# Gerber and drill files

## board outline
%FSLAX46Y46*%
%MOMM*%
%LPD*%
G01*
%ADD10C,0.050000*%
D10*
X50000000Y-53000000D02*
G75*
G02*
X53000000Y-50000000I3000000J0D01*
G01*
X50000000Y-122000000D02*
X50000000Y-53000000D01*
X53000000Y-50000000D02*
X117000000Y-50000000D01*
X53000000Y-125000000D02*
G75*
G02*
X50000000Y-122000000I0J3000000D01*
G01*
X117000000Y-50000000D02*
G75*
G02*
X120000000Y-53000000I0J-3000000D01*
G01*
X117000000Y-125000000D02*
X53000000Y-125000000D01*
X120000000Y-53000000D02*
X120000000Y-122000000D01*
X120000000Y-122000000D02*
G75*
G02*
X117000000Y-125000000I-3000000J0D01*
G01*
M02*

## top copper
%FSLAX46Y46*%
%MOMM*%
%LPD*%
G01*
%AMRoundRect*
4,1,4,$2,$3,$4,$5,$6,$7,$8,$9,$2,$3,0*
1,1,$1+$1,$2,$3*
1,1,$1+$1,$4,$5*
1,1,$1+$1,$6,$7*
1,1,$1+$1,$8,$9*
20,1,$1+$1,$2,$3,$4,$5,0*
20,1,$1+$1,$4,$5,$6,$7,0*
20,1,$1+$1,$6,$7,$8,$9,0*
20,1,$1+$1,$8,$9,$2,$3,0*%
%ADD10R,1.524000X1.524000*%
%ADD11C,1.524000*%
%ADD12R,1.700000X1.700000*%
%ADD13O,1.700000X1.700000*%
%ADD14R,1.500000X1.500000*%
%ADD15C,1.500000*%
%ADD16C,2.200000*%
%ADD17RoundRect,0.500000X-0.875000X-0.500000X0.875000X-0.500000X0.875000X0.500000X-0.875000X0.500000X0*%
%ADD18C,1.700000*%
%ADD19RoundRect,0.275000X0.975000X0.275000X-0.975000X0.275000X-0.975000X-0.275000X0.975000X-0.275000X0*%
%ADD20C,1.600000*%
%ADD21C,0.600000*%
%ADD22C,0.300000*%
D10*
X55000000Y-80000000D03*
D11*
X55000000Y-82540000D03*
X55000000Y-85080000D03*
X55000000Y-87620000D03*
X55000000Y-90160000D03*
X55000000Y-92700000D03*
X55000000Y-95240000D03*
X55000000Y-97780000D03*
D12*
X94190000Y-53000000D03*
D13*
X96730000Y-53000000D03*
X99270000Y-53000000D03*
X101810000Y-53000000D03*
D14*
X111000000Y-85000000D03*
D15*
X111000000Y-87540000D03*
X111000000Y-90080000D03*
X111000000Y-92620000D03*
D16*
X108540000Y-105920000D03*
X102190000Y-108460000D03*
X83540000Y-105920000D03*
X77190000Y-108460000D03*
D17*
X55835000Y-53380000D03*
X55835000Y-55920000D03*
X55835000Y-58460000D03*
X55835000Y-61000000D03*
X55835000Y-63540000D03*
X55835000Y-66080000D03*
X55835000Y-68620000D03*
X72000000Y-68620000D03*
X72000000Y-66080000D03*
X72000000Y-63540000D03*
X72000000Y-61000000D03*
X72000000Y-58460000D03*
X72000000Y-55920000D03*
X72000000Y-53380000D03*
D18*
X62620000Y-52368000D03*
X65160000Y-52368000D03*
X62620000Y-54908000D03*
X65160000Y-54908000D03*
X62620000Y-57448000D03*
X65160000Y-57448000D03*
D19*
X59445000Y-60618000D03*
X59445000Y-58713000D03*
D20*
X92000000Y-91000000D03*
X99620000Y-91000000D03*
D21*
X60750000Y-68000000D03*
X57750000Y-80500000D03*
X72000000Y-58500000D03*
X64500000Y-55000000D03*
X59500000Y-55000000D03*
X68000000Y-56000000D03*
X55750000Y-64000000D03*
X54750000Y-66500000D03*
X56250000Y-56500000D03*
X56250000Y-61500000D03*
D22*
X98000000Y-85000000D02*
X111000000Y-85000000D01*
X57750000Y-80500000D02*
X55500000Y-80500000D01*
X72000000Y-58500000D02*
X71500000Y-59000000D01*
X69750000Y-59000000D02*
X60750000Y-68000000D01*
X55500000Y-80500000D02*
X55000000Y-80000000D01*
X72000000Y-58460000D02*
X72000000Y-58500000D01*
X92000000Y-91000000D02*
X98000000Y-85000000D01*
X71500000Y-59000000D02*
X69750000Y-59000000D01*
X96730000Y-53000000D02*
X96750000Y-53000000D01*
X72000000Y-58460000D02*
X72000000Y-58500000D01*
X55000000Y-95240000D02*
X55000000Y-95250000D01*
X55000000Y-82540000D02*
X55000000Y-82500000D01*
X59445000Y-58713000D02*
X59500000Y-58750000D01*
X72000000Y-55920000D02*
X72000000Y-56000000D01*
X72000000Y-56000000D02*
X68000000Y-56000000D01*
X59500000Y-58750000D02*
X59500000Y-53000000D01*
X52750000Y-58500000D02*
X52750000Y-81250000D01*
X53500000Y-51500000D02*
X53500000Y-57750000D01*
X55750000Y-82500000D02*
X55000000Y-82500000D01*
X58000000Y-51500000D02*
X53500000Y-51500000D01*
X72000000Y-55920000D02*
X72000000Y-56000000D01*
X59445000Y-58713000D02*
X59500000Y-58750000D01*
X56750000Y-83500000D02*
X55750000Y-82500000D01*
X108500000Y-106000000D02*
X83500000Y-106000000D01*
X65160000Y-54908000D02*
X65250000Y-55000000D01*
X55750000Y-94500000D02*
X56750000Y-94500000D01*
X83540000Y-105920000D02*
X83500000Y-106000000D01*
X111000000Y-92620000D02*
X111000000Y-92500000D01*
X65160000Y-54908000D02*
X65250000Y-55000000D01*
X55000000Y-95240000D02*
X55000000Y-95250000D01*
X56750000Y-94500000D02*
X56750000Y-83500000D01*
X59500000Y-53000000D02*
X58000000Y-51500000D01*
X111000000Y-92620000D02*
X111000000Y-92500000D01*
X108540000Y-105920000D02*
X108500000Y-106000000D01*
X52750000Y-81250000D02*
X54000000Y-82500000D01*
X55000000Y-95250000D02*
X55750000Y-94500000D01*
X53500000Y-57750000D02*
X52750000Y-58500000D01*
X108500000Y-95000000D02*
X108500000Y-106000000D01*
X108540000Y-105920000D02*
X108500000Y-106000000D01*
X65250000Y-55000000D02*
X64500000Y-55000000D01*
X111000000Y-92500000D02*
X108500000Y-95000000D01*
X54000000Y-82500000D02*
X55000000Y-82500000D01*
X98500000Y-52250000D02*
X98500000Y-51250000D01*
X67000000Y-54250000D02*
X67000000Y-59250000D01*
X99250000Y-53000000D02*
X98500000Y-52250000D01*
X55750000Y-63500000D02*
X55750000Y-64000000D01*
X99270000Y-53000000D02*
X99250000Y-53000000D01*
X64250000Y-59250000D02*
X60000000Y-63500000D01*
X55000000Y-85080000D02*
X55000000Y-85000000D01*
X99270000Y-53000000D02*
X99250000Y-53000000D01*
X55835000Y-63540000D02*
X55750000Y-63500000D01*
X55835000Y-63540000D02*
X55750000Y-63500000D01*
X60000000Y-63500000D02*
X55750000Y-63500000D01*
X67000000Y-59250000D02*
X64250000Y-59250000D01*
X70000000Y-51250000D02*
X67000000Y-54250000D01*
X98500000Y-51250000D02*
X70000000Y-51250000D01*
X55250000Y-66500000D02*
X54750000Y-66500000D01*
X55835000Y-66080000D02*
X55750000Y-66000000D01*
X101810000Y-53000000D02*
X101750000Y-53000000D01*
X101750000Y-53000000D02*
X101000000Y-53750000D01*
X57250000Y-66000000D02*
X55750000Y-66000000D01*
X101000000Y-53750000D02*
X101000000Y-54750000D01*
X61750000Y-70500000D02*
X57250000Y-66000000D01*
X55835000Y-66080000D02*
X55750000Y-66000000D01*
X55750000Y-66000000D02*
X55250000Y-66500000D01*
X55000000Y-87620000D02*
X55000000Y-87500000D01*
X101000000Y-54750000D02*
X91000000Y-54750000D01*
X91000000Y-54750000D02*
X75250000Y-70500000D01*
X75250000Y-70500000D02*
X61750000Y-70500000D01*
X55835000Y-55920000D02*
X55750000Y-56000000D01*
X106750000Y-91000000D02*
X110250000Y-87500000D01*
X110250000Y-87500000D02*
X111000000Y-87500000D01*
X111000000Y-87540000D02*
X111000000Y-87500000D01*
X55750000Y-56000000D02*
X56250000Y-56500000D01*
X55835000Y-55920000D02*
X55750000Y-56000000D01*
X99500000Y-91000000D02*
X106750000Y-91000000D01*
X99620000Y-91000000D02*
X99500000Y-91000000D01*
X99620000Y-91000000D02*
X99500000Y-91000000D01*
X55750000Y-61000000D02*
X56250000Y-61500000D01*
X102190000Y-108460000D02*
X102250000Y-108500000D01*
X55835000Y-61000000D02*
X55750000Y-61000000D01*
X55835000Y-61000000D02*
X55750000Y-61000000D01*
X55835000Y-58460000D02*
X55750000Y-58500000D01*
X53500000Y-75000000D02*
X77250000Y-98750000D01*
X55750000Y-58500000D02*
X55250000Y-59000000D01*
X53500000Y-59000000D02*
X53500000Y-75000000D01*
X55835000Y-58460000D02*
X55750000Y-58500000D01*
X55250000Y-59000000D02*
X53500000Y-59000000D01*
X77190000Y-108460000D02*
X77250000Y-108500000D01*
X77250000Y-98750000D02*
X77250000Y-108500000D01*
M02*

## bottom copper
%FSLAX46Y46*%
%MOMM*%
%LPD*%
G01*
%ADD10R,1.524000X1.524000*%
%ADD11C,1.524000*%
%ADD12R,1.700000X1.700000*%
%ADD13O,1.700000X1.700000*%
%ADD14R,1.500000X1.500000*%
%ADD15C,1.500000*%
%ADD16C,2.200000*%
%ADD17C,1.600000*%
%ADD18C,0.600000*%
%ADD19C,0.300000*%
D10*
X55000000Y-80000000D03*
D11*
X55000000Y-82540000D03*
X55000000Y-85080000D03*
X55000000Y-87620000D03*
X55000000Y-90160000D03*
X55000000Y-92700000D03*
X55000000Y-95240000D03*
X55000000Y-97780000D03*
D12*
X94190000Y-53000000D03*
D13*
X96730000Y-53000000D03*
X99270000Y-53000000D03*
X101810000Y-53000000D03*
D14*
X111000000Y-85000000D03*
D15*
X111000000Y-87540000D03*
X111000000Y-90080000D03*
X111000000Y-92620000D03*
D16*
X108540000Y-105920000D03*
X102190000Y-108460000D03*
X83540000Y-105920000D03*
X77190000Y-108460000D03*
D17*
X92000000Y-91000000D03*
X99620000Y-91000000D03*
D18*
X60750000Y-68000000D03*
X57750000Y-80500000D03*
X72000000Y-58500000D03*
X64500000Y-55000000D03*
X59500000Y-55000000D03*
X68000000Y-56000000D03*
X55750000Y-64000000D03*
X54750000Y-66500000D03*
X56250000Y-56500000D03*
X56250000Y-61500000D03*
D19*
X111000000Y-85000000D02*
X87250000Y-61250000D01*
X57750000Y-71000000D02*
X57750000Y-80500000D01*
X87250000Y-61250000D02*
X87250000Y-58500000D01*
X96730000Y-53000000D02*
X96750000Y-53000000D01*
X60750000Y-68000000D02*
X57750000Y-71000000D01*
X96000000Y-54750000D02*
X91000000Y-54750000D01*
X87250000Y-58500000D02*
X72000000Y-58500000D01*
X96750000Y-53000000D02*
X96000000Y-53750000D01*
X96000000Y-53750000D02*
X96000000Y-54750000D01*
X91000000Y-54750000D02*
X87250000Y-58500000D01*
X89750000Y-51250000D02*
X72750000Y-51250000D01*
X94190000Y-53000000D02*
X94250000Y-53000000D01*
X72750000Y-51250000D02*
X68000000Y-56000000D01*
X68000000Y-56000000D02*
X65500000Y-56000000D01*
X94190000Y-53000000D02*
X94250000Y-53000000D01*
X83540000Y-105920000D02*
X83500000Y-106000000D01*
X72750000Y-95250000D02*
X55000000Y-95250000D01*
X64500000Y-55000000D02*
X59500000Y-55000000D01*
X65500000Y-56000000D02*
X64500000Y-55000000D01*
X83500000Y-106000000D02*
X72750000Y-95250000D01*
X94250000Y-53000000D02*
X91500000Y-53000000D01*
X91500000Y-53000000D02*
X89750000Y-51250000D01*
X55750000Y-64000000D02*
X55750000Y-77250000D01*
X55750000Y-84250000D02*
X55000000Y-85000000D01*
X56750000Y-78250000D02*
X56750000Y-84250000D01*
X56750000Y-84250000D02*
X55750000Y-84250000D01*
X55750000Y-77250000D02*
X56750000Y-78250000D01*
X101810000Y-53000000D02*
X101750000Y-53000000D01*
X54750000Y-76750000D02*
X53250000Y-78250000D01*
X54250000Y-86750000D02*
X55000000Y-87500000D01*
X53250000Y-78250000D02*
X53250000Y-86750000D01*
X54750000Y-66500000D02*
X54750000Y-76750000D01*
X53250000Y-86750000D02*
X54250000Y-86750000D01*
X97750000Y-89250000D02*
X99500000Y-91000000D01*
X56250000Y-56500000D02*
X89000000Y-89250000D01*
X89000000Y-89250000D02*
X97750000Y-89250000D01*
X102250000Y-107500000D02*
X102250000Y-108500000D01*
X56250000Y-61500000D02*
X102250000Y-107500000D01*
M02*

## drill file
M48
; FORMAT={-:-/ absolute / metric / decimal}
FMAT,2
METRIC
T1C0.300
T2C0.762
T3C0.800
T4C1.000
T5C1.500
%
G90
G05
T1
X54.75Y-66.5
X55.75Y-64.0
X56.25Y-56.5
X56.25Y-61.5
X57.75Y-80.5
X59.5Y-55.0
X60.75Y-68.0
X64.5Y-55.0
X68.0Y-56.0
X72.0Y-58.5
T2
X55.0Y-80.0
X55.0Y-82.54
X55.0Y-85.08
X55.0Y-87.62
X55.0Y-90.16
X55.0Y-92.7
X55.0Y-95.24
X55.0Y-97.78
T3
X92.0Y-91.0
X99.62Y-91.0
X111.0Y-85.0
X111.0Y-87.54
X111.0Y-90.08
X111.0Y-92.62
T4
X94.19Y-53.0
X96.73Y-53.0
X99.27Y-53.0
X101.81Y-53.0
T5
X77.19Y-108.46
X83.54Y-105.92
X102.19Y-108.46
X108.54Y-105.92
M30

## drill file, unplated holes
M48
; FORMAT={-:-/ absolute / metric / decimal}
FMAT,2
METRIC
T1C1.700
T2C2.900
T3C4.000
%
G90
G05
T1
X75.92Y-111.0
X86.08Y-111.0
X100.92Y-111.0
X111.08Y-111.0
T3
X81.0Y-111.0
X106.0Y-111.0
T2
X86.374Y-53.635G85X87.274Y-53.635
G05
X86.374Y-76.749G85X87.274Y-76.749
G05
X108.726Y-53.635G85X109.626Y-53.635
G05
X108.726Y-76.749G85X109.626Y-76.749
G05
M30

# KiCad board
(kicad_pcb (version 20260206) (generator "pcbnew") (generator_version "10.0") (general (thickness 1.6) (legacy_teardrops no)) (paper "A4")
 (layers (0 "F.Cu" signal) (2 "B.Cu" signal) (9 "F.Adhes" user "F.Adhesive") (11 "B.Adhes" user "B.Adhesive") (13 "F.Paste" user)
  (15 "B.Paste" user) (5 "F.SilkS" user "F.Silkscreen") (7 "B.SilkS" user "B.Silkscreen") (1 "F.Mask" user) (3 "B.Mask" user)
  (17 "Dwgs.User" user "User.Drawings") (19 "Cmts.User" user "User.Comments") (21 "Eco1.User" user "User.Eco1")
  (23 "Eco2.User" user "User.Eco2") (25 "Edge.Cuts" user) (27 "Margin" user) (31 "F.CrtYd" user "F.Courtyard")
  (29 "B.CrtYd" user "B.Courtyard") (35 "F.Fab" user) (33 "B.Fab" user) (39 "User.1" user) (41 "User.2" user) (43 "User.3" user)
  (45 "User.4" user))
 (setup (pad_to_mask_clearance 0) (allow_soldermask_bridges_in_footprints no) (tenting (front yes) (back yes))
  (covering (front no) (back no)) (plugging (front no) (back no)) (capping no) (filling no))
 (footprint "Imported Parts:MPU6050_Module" (layer "F.Cu") (at 55 80)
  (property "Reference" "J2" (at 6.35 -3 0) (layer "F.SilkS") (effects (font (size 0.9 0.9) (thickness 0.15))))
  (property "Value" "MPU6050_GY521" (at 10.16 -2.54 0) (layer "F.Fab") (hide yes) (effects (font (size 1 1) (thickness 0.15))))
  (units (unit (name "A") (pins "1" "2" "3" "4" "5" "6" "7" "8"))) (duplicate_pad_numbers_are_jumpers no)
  (pad "1" thru_hole rect (at 0 0) (size 1.524 1.524) (drill 0.762) (layers "*.Cu" "*.Mask") (remove_unused_layers no) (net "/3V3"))
  (pad "2" thru_hole circle (at 0 2.54) (size 1.524 1.524) (drill 0.762) (layers "*.Cu" "*.Mask") (remove_unused_layers no) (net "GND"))
  (pad "3" thru_hole circle (at 0 5.08) (size 1.524 1.524) (drill 0.762) (layers "*.Cu" "*.Mask") (remove_unused_layers no) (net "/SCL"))
  (pad "4" thru_hole circle (at 0 7.62) (size 1.524 1.524) (drill 0.762) (layers "*.Cu" "*.Mask") (remove_unused_layers no) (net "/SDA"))
  (pad "5" thru_hole circle (at 0 10.16) (size 1.524 1.524) (drill 0.762) (layers "*.Cu" "*.Mask") (remove_unused_layers no)
   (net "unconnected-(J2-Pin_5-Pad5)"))
  (pad "6" thru_hole circle (at 0 12.7) (size 1.524 1.524) (drill 0.762) (layers "*.Cu" "*.Mask") (remove_unused_layers no)
   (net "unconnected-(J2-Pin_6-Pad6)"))
  (pad "7" thru_hole circle (at 0 15.24) (size 1.524 1.524) (drill 0.762) (layers "*.Cu" "*.Mask") (remove_unused_layers no) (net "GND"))
  (pad "8" thru_hole circle (at 0 17.78) (size 1.524 1.524) (drill 0.762) (layers "*.Cu" "*.Mask") (remove_unused_layers no)
   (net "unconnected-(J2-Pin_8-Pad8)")))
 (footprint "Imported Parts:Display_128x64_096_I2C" (layer "F.Cu") (at 98 53)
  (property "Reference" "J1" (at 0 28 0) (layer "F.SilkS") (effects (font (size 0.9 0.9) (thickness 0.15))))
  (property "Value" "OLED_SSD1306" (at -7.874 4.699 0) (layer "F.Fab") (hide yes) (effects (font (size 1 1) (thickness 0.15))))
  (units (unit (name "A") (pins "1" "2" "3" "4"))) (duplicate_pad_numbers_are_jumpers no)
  (pad "" np_thru_hole oval (at -11.176 0.635) (size 3.8 2.9) (drill oval 3.8 2.9) (layers "*.Cu" "*.Mask"))
  (pad "" np_thru_hole oval (at -11.176 23.749) (size 3.8 2.9) (drill oval 3.8 2.9) (layers "*.Cu" "*.Mask"))
  (pad "" np_thru_hole oval (at 11.176 0.635) (size 3.8 2.9) (drill oval 3.8 2.9) (layers "*.Cu" "*.Mask"))
  (pad "" np_thru_hole oval (at 11.176 23.749) (size 3.8 2.9) (drill oval 3.8 2.9) (layers "*.Cu" "*.Mask"))
  (pad "1" thru_hole rect (at -3.81 0 90) (size 1.7 1.7) (drill 1) (layers "*.Cu" "*.Mask") (remove_unused_layers no) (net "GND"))
  (pad "2" thru_hole oval (at -1.27 0 90) (size 1.7 1.7) (drill 1) (layers "*.Cu" "*.Mask") (remove_unused_layers no) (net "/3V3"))
  (pad "3" thru_hole oval (at 1.27 0 90) (size 1.7 1.7) (drill 1) (layers "*.Cu" "*.Mask") (remove_unused_layers no) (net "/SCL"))
  (pad "4" thru_hole oval (at 3.81 0 90) (size 1.7 1.7) (drill 1) (layers "*.Cu" "*.Mask") (remove_unused_layers no) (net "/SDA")))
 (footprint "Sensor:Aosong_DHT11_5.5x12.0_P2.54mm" (layer "F.Cu") (at 111 85)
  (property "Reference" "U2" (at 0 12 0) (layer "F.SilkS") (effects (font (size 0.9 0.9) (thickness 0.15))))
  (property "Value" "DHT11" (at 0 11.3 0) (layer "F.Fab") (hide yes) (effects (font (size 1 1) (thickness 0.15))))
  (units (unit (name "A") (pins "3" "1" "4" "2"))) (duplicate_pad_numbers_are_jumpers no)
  (pad "1" thru_hole rect (at 0 0) (size 1.5 1.5) (drill 0.8) (layers "*.Cu" "*.Mask") (remove_unused_layers no) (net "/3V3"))
  (pad "2" thru_hole circle (at 0 2.54) (size 1.5 1.5) (drill 0.8) (layers "*.Cu" "*.Mask") (remove_unused_layers no) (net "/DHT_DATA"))
  (pad "3" thru_hole circle (at 0 5.08) (size 1.5 1.5) (drill 0.8) (layers "*.Cu" "*.Mask") (remove_unused_layers no)
   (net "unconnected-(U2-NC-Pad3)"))
  (pad "4" thru_hole circle (at 0 7.62) (size 1.5 1.5) (drill 0.8) (layers "*.Cu" "*.Mask") (remove_unused_layers no) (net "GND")))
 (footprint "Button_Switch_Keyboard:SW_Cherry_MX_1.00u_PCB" (layer "F.Cu") (at 108.54 105.92)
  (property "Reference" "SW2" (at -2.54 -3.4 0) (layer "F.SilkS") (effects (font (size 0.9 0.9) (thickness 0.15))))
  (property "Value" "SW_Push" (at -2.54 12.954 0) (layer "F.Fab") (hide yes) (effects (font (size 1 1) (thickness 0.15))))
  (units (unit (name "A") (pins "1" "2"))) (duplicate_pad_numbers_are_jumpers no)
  (pad "" np_thru_hole circle (at -7.62 5.08) (size 1.7 1.7) (drill 1.7) (layers "*.Cu" "*.Mask"))
  (pad "" np_thru_hole circle (at -2.54 5.08) (size 4 4) (drill 4) (layers "*.Cu" "*.Mask"))
  (pad "" np_thru_hole circle (at 2.54 5.08) (size 1.7 1.7) (drill 1.7) (layers "*.Cu" "*.Mask"))
  (pad "1" thru_hole circle (at 0 0) (size 2.2 2.2) (drill 1.5) (layers "*.Cu" "*.Mask") (remove_unused_layers no) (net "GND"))
  (pad "2" thru_hole circle (at -6.35 2.54) (size 2.2 2.2) (drill 1.5) (layers "*.Cu" "*.Mask") (remove_unused_layers no)
   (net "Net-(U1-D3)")))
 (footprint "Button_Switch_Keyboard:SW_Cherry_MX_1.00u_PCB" (layer "F.Cu") (at 83.54 105.92)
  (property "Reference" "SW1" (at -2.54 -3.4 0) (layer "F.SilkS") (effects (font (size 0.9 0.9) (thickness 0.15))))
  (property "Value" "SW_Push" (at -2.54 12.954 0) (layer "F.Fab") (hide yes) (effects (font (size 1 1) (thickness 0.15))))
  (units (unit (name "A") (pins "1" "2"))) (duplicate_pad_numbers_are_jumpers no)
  (pad "" np_thru_hole circle (at -7.62 5.08) (size 1.7 1.7) (drill 1.7) (layers "*.Cu" "*.Mask"))
  (pad "" np_thru_hole circle (at -2.54 5.08) (size 4 4) (drill 4) (layers "*.Cu" "*.Mask"))
  (pad "" np_thru_hole circle (at 2.54 5.08) (size 1.7 1.7) (drill 1.7) (layers "*.Cu" "*.Mask"))
  (pad "1" thru_hole circle (at 0 0) (size 2.2 2.2) (drill 1.5) (layers "*.Cu" "*.Mask") (remove_unused_layers no) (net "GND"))
  (pad "2" thru_hole circle (at -6.35 2.54) (size 2.2 2.2) (drill 1.5) (layers "*.Cu" "*.Mask") (remove_unused_layers no)
   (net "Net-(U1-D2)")))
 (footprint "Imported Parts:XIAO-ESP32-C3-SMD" (layer "F.Cu") (at 55 71.5)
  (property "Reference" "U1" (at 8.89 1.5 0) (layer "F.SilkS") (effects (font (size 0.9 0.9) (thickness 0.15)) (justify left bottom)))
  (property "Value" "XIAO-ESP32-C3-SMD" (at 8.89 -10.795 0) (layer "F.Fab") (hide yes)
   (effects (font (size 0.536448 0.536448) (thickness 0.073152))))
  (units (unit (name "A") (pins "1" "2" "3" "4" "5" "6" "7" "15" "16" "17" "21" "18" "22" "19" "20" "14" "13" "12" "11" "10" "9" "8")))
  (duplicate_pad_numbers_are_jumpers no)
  (pad "1" smd roundrect (at 0.835 -18.12) (size 2.75 2) (layers "F.Cu" "F.Mask" "F.Paste") (roundrect_rratio 0.25)
   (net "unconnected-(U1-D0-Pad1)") (solder_mask_margin 0.0508) (thermal_bridge_angle 45))
  (pad "2" smd roundrect (at 0.835 -15.58) (size 2.75 2) (layers "F.Cu" "F.Mask" "F.Paste") (roundrect_rratio 0.25) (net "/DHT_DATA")
   (solder_mask_margin 0.0508) (thermal_bridge_angle 45))
  (pad "3" smd roundrect (at 0.835 -13.04) (size 2.75 2) (layers "F.Cu" "F.Mask" "F.Paste") (roundrect_rratio 0.25) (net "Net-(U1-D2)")
   (solder_mask_margin 0.0508) (thermal_bridge_angle 45))
  (pad "4" smd roundrect (at 0.835 -10.5) (size 2.75 2) (layers "F.Cu" "F.Mask" "F.Paste") (roundrect_rratio 0.25) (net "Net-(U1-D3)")
   (solder_mask_margin 0.0508) (thermal_bridge_angle 45))
  (pad "5" smd roundrect (at 0.835 -7.96) (size 2.75 2) (layers "F.Cu" "F.Mask" "F.Paste") (roundrect_rratio 0.25) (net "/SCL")
   (solder_mask_margin 0.0508) (thermal_bridge_angle 45))
  (pad "6" smd roundrect (at 0.835 -5.42) (size 2.75 2) (layers "F.Cu" "F.Mask" "F.Paste") (roundrect_rratio 0.25) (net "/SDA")
   (solder_mask_margin 0.0508) (thermal_bridge_angle 45))
  (pad "7" smd roundrect (at 0.835 -2.88) (size 2.75 2) (layers "F.Cu" "F.Mask" "F.Paste") (roundrect_rratio 0.25)
   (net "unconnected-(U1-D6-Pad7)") (solder_mask_margin 0.0508) (thermal_bridge_angle 45))
  (pad "8" smd roundrect (at 17 -2.88) (size 2.75 2) (layers "F.Cu" "F.Mask" "F.Paste") (roundrect_rratio 0.25)
   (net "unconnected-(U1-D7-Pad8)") (solder_mask_margin 0.0508) (thermal_bridge_angle 45))
  (pad "9" smd roundrect (at 17 -5.42) (size 2.75 2) (layers "F.Cu" "F.Mask" "F.Paste") (roundrect_rratio 0.25)
   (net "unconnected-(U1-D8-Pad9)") (solder_mask_margin 0.0508) (thermal_bridge_angle 45))
  (pad "10" smd roundrect (at 17 -7.96) (size 2.75 2) (layers "F.Cu" "F.Mask" "F.Paste") (roundrect_rratio 0.25)
   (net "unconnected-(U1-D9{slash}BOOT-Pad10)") (solder_mask_margin 0.0508) (thermal_bridge_angle 45))
  (pad "11" smd roundrect (at 17 -10.5) (size 2.75 2) (layers "F.Cu" "F.Mask" "F.Paste") (roundrect_rratio 0.25)
   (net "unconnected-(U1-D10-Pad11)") (solder_mask_margin 0.0508) (thermal_bridge_angle 45))
  (pad "12" smd roundrect (at 17 -13.04) (size 2.75 2) (layers "F.Cu" "F.Mask" "F.Paste") (roundrect_rratio 0.25) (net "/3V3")
   (solder_mask_margin 0.0508) (thermal_bridge_angle 45))
  (pad "13" smd roundrect (at 17 -15.58) (size 2.75 2) (layers "F.Cu" "F.Mask" "F.Paste") (roundrect_rratio 0.25) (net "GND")
   (solder_mask_margin 0.0508) (thermal_bridge_angle 45))
  (pad "14" smd roundrect (at 17 -18.12) (size 2.75 2) (layers "F.Cu" "F.Mask" "F.Paste") (roundrect_rratio 0.25)
   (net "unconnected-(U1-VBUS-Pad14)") (solder_mask_margin 0.0508) (thermal_bridge_angle 45))
  (pad "15" smd circle (at 7.62 -19.132) (size 1.7 1.7) (layers "F.Cu" "F.Mask" "F.Paste") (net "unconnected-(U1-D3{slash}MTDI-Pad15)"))
  (pad "16" smd circle (at 10.16 -19.132) (size 1.7 1.7) (layers "F.Cu" "F.Mask" "F.Paste") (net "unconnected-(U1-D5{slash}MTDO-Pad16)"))
  (pad "17" smd circle (at 7.62 -16.592) (size 1.7 1.7) (layers "F.Cu" "F.Mask" "F.Paste") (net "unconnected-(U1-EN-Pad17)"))
  (pad "18" smd circle (at 10.16 -16.592) (size 1.7 1.7) (layers "F.Cu" "F.Mask" "F.Paste") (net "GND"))
  (pad "19" smd circle (at 7.62 -14.052) (size 1.7 1.7) (layers "F.Cu" "F.Mask" "F.Paste") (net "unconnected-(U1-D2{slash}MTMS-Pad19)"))
  (pad "20" smd circle (at 10.16 -14.052) (size 1.7 1.7) (layers "F.Cu" "F.Mask" "F.Paste") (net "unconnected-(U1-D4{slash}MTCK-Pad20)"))
  (pad "21" smd roundrect (at 4.445 -10.882 180) (size 2.5 1.1) (layers "F.Cu" "F.Mask" "F.Paste") (roundrect_rratio 0.25)
   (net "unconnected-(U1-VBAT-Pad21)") (thermal_bridge_angle 45))
  (pad "22" smd roundrect (at 4.445 -12.787 180) (size 2.5 1.1) (layers "F.Cu" "F.Mask" "F.Paste") (roundrect_rratio 0.25) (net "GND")
   (thermal_bridge_angle 45)))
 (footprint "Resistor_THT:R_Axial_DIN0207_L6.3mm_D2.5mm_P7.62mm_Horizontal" (layer "F.Cu") (at 92 91)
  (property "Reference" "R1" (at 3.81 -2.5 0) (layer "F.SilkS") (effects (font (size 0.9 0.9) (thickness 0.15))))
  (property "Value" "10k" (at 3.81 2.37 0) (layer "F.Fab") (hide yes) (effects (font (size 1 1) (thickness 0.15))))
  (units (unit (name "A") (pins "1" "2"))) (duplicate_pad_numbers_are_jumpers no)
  (pad "1" thru_hole circle (at 0 0) (size 1.6 1.6) (drill 0.8) (layers "*.Cu" "*.Mask") (remove_unused_layers no) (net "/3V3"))
  (pad "2" thru_hole circle (at 7.62 0) (size 1.6 1.6) (drill 0.8) (layers "*.Cu" "*.Mask") (remove_unused_layers no) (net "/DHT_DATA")))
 (gr_arc (start 50 53) (mid 50.87868 50.87868) (end 53 50) (stroke (width 0.05) (type default)) (layer "Edge.Cuts"))
 (gr_line (start 50 122) (end 50 53) (stroke (width 0.05) (type default)) (layer "Edge.Cuts"))
 (gr_line (start 53 50) (end 117 50) (stroke (width 0.05) (type default)) (layer "Edge.Cuts"))
 (gr_arc (start 53 125) (mid 50.87868 124.12132) (end 50 122) (stroke (width 0.05) (type default)) (layer "Edge.Cuts"))
 (gr_arc (start 117 50) (mid 119.12132 50.87868) (end 120 53) (stroke (width 0.05) (type default)) (layer "Edge.Cuts"))
 (gr_line (start 117 125) (end 53 125) (stroke (width 0.05) (type default)) (layer "Edge.Cuts"))
 (gr_line (start 120 53) (end 120 122) (stroke (width 0.05) (type default)) (layer "Edge.Cuts"))
 (gr_arc (start 120 122) (mid 119.12132 124.12132) (end 117 125) (stroke (width 0.05) (type default)) (layer "Edge.Cuts"))
 (segment (start 98 85) (end 111 85) (width 0.3) (layer "F.Cu") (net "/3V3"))
 (segment (start 57.75 80.5) (end 55.5 80.5) (width 0.3) (layer "F.Cu") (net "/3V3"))
 (segment (start 72 58.5) (end 71.5 59) (width 0.3) (layer "F.Cu") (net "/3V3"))
 (segment (start 69.75 59) (end 60.75 68) (width 0.3) (layer "F.Cu") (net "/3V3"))
 (segment (start 55.5 80.5) (end 55 80) (width 0.3) (layer "F.Cu") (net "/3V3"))
 (segment (start 72 58.46) (end 72 58.5) (width 0.3) (layer "F.Cu") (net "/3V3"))
 (segment (start 92 91) (end 98 85) (width 0.3) (layer "F.Cu") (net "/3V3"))
 (segment (start 71.5 59) (end 69.75 59) (width 0.3) (layer "F.Cu") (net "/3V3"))
 (segment (start 96.73 53) (end 96.75 53) (width 0.3) (layer "F.Cu") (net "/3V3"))
 (segment (start 72 58.46) (end 72 58.5) (width 0.3) (layer "F.Cu") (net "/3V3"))
 (via (at 60.75 68) (size 0.6) (drill 0.3) (layers "F.Cu" "B.Cu") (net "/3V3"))
 (via (at 57.75 80.5) (size 0.6) (drill 0.3) (layers "F.Cu" "B.Cu") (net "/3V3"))
 (via (at 72 58.5) (size 0.6) (drill 0.3) (layers "F.Cu" "B.Cu") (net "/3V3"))
 (segment (start 111 85) (end 87.25 61.25) (width 0.3) (layer "B.Cu") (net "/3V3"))
 (segment (start 57.75 71) (end 57.75 80.5) (width 0.3) (layer "B.Cu") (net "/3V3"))
 (segment (start 87.25 61.25) (end 87.25 58.5) (width 0.3) (layer "B.Cu") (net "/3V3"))
 (segment (start 96.73 53) (end 96.75 53) (width 0.3) (layer "B.Cu") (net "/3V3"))
 (segment (start 60.75 68) (end 57.75 71) (width 0.3) (layer "B.Cu") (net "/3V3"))
 (segment (start 96 54.75) (end 91 54.75) (width 0.3) (layer "B.Cu") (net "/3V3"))
 (segment (start 87.25 58.5) (end 72 58.5) (width 0.3) (layer "B.Cu") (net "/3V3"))
 (segment (start 96.75 53) (end 96 53.75) (width 0.3) (layer "B.Cu") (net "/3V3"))
 (segment (start 96 53.75) (end 96 54.75) (width 0.3) (layer "B.Cu") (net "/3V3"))
 (segment (start 91 54.75) (end 87.25 58.5) (width 0.3) (layer "B.Cu") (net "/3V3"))
 (segment (start 55 95.24) (end 55 95.25) (width 0.3) (layer "F.Cu") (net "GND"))
 (segment (start 55 82.54) (end 55 82.5) (width 0.3) (layer "F.Cu") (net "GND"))
 (segment (start 59.445 58.713) (end 59.5 58.75) (width 0.3) (layer "F.Cu") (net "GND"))
 (segment (start 72 55.92) (end 72 56) (width 0.3) (layer "F.Cu") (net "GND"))
 (segment (start 72 56) (end 68 56) (width 0.3) (layer "F.Cu") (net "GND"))
 (segment (start 59.5 58.75) (end 59.5 53) (width 0.3) (layer "F.Cu") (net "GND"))
 (segment (start 52.75 58.5) (end 52.75 81.25) (width 0.3) (layer "F.Cu") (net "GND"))
 (segment (start 53.5 51.5) (end 53.5 57.75) (width 0.3) (layer "F.Cu") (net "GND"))
 (segment (start 55.75 82.5) (end 55 82.5) (width 0.3) (layer "F.Cu") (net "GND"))
 (segment (start 58 51.5) (end 53.5 51.5) (width 0.3) (layer "F.Cu") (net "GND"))
 (segment (start 72 55.92) (end 72 56) (width 0.3) (layer "F.Cu") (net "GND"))
 (segment (start 59.445 58.713) (end 59.5 58.75) (width 0.3) (layer "F.Cu") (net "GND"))
 (segment (start 56.75 83.5) (end 55.75 82.5) (width 0.3) (layer "F.Cu") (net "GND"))
 (segment (start 108.5 106) (end 83.5 106) (width 0.3) (layer "F.Cu") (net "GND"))
 (segment (start 65.16 54.908) (end 65.25 55) (width 0.3) (layer "F.Cu") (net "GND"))
 (segment (start 55.75 94.5) (end 56.75 94.5) (width 0.3) (layer "F.Cu") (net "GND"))
 (segment (start 83.54 105.92) (end 83.5 106) (width 0.3) (layer "F.Cu") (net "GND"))
 (segment (start 111 92.62) (end 111 92.5) (width 0.3) (layer "F.Cu") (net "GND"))
 (segment (start 65.16 54.908) (end 65.25 55) (width 0.3) (layer "F.Cu") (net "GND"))
 (segment (start 55 95.24) (end 55 95.25) (width 0.3) (layer "F.Cu") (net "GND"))
 (segment (start 56.75 94.5) (end 56.75 83.5) (width 0.3) (layer "F.Cu") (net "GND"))
 (segment (start 59.5 53) (end 58 51.5) (width 0.3) (layer "F.Cu") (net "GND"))
 (segment (start 111 92.62) (end 111 92.5) (width 0.3) (layer "F.Cu") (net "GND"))
 (segment (start 108.54 105.92) (end 108.5 106) (width 0.3) (layer "F.Cu") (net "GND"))
 (segment (start 52.75 81.25) (end 54 82.5) (width 0.3) (layer "F.Cu") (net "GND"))
 (segment (start 55 95.25) (end 55.75 94.5) (width 0.3) (layer "F.Cu") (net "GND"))
 (segment (start 53.5 57.75) (end 52.75 58.5) (width 0.3) (layer "F.Cu") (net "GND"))
 (segment (start 108.5 95) (end 108.5 106) (width 0.3) (layer "F.Cu") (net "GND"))
 (segment (start 108.54 105.92) (end 108.5 106) (width 0.3) (layer "F.Cu") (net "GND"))
 (segment (start 65.25 55) (end 64.5 55) (width 0.3) (layer "F.Cu") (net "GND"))
 (segment (start 111 92.5) (end 108.5 95) (width 0.3) (layer "F.Cu") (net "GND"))
 (segment (start 54 82.5) (end 55 82.5) (width 0.3) (layer "F.Cu") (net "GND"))
 (via (at 64.5 55) (size 0.6) (drill 0.3) (layers "F.Cu" "B.Cu") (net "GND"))
 (via (at 59.5 55) (size 0.6) (drill 0.3) (layers "F.Cu" "B.Cu") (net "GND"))
 (via (at 68 56) (size 0.6) (drill 0.3) (layers "F.Cu" "B.Cu") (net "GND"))
 (segment (start 89.75 51.25) (end 72.75 51.25) (width 0.3) (layer "B.Cu") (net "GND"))
 (segment (start 94.19 53) (end 94.25 53) (width 0.3) (layer "B.Cu") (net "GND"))
 (segment (start 72.75 51.25) (end 68 56) (width 0.3) (layer "B.Cu") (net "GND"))
 (segment (start 68 56) (end 65.5 56) (width 0.3) (layer "B.Cu") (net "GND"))
 (segment (start 94.19 53) (end 94.25 53) (width 0.3) (layer "B.Cu") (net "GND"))
 (segment (start 83.54 105.92) (end 83.5 106) (width 0.3) (layer "B.Cu") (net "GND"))
 (segment (start 72.75 95.25) (end 55 95.25) (width 0.3) (layer "B.Cu") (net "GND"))
 (segment (start 64.5 55) (end 59.5 55) (width 0.3) (layer "B.Cu") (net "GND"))
 (segment (start 65.5 56) (end 64.5 55) (width 0.3) (layer "B.Cu") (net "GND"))
 (segment (start 83.5 106) (end 72.75 95.25) (width 0.3) (layer "B.Cu") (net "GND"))
 (segment (start 94.25 53) (end 91.5 53) (width 0.3) (layer "B.Cu") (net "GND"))
 (segment (start 91.5 53) (end 89.75 51.25) (width 0.3) (layer "B.Cu") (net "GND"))
 (segment (start 98.5 52.25) (end 98.5 51.25) (width 0.3) (layer "F.Cu") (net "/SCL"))
 (segment (start 67 54.25) (end 67 59.25) (width 0.3) (layer "F.Cu") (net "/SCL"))
 (segment (start 99.25 53) (end 98.5 52.25) (width 0.3) (layer "F.Cu") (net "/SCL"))
 (segment (start 55.75 63.5) (end 55.75 64) (width 0.3) (layer "F.Cu") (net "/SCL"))
 (segment (start 99.27 53) (end 99.25 53) (width 0.3) (layer "F.Cu") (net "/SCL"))
 (segment (start 64.25 59.25) (end 60 63.5) (width 0.3) (layer "F.Cu") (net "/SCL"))
 (segment (start 55 85.08) (end 55 85) (width 0.3) (layer "F.Cu") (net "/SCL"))
 (segment (start 99.27 53) (end 99.25 53) (width 0.3) (layer "F.Cu") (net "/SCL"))
 (segment (start 55.835 63.54) (end 55.75 63.5) (width 0.3) (layer "F.Cu") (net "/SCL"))
 (segment (start 55.835 63.54) (end 55.75 63.5) (width 0.3) (layer "F.Cu") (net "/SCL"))
 (segment (start 60 63.5) (end 55.75 63.5) (width 0.3) (layer "F.Cu") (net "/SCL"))
 (segment (start 67 59.25) (end 64.25 59.25) (width 0.3) (layer "F.Cu") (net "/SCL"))
 (segment (start 70 51.25) (end 67 54.25) (width 0.3) (layer "F.Cu") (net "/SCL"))
 (segment (start 98.5 51.25) (end 70 51.25) (width 0.3) (layer "F.Cu") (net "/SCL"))
 (via (at 55.75 64) (size 0.6) (drill 0.3) (layers "F.Cu" "B.Cu") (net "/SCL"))
 (segment (start 55.75 64) (end 55.75 77.25) (width 0.3) (layer "B.Cu") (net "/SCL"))
 (segment (start 55.75 84.25) (end 55 85) (width 0.3) (layer "B.Cu") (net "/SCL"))
 (segment (start 56.75 78.25) (end 56.75 84.25) (width 0.3) (layer "B.Cu") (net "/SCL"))
 (segment (start 56.75 84.25) (end 55.75 84.25) (width 0.3) (layer "B.Cu") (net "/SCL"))
 (segment (start 55.75 77.25) (end 56.75 78.25) (width 0.3) (layer "B.Cu") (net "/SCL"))
 (segment (start 55.25 66.5) (end 54.75 66.5) (width 0.3) (layer "F.Cu") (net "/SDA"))
 (segment (start 55.835 66.08) (end 55.75 66) (width 0.3) (layer "F.Cu") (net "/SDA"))
 (segment (start 101.81 53) (end 101.75 53) (width 0.3) (layer "F.Cu") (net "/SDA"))
 (segment (start 101.75 53) (end 101 53.75) (width 0.3) (layer "F.Cu") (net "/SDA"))
 (segment (start 57.25 66) (end 55.75 66) (width 0.3) (layer "F.Cu") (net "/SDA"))
 (segment (start 101 53.75) (end 101 54.75) (width 0.3) (layer "F.Cu") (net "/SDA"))
 (segment (start 61.75 70.5) (end 57.25 66) (width 0.3) (layer "F.Cu") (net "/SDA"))
 (segment (start 55.835 66.08) (end 55.75 66) (width 0.3) (layer "F.Cu") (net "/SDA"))
 (segment (start 55.75 66) (end 55.25 66.5) (width 0.3) (layer "F.Cu") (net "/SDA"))
 (segment (start 55 87.62) (end 55 87.5) (width 0.3) (layer "F.Cu") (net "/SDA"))
 (segment (start 101 54.75) (end 91 54.75) (width 0.3) (layer "F.Cu") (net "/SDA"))
 (segment (start 91 54.75) (end 75.25 70.5) (width 0.3) (layer "F.Cu") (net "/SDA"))
 (segment (start 75.25 70.5) (end 61.75 70.5) (width 0.3) (layer "F.Cu") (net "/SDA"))
 (via (at 54.75 66.5) (size 0.6) (drill 0.3) (layers "F.Cu" "B.Cu") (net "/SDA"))
 (segment (start 101.81 53) (end 101.75 53) (width 0.3) (layer "B.Cu") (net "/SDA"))
 (segment (start 54.75 76.75) (end 53.25 78.25) (width 0.3) (layer "B.Cu") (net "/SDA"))
 (segment (start 54.25 86.75) (end 55 87.5) (width 0.3) (layer "B.Cu") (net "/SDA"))
 (segment (start 53.25 78.25) (end 53.25 86.75) (width 0.3) (layer "B.Cu") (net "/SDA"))
 (segment (start 54.75 66.5) (end 54.75 76.75) (width 0.3) (layer "B.Cu") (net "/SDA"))
 (segment (start 53.25 86.75) (end 54.25 86.75) (width 0.3) (layer "B.Cu") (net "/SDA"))
 (segment (start 55.835 55.92) (end 55.75 56) (width 0.3) (layer "F.Cu") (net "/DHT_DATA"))
 (segment (start 106.75 91) (end 110.25 87.5) (width 0.3) (layer "F.Cu") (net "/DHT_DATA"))
 (segment (start 110.25 87.5) (end 111 87.5) (width 0.3) (layer "F.Cu") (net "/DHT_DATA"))
 (segment (start 111 87.54) (end 111 87.5) (width 0.3) (layer "F.Cu") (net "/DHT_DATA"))
 (segment (start 55.75 56) (end 56.25 56.5) (width 0.3) (layer "F.Cu") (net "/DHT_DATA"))
 (segment (start 55.835 55.92) (end 55.75 56) (width 0.3) (layer "F.Cu") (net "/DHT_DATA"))
 (segment (start 99.5 91) (end 106.75 91) (width 0.3) (layer "F.Cu") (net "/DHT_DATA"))
 (segment (start 99.62 91) (end 99.5 91) (width 0.3) (layer "F.Cu") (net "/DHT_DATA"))
 (segment (start 99.62 91) (end 99.5 91) (width 0.3) (layer "F.Cu") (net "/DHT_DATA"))
 (via (at 56.25 56.5) (size 0.6) (drill 0.3) (layers "F.Cu" "B.Cu") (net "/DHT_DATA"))
 (segment (start 97.75 89.25) (end 99.5 91) (width 0.3) (layer "B.Cu") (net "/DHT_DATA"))
 (segment (start 56.25 56.5) (end 89 89.25) (width 0.3) (layer "B.Cu") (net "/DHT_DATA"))
 (segment (start 89 89.25) (end 97.75 89.25) (width 0.3) (layer "B.Cu") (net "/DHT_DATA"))
 (segment (start 55.75 61) (end 56.25 61.5) (width 0.3) (layer "F.Cu") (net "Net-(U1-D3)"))
 (segment (start 102.19 108.46) (end 102.25 108.5) (width 0.3) (layer "F.Cu") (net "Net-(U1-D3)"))
 (segment (start 55.835 61) (end 55.75 61) (width 0.3) (layer "F.Cu") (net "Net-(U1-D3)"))
 (segment (start 55.835 61) (end 55.75 61) (width 0.3) (layer "F.Cu") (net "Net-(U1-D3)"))
 (via (at 56.25 61.5) (size 0.6) (drill 0.3) (layers "F.Cu" "B.Cu") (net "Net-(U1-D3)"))
 (segment (start 102.25 107.5) (end 102.25 108.5) (width 0.3) (layer "B.Cu") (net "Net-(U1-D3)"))
 (segment (start 56.25 61.5) (end 102.25 107.5) (width 0.3) (layer "B.Cu") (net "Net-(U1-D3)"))
 (segment (start 55.835 58.46) (end 55.75 58.5) (width 0.3) (layer "F.Cu") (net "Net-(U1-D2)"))
 (segment (start 53.5 75) (end 77.25 98.75) (width 0.3) (layer "F.Cu") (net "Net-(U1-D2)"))
 (segment (start 55.75 58.5) (end 55.25 59) (width 0.3) (layer "F.Cu") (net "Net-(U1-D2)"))
 (segment (start 53.5 59) (end 53.5 75) (width 0.3) (layer "F.Cu") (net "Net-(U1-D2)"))
 (segment (start 55.835 58.46) (end 55.75 58.5) (width 0.3) (layer "F.Cu") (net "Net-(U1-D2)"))
 (segment (start 55.25 59) (end 53.5 59) (width 0.3) (layer "F.Cu") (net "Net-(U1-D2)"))
 (segment (start 77.19 108.46) (end 77.25 108.5) (width 0.3) (layer "F.Cu") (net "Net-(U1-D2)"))
 (segment (start 77.25 98.75) (end 77.25 108.5) (width 0.3) (layer "F.Cu") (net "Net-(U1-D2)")))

